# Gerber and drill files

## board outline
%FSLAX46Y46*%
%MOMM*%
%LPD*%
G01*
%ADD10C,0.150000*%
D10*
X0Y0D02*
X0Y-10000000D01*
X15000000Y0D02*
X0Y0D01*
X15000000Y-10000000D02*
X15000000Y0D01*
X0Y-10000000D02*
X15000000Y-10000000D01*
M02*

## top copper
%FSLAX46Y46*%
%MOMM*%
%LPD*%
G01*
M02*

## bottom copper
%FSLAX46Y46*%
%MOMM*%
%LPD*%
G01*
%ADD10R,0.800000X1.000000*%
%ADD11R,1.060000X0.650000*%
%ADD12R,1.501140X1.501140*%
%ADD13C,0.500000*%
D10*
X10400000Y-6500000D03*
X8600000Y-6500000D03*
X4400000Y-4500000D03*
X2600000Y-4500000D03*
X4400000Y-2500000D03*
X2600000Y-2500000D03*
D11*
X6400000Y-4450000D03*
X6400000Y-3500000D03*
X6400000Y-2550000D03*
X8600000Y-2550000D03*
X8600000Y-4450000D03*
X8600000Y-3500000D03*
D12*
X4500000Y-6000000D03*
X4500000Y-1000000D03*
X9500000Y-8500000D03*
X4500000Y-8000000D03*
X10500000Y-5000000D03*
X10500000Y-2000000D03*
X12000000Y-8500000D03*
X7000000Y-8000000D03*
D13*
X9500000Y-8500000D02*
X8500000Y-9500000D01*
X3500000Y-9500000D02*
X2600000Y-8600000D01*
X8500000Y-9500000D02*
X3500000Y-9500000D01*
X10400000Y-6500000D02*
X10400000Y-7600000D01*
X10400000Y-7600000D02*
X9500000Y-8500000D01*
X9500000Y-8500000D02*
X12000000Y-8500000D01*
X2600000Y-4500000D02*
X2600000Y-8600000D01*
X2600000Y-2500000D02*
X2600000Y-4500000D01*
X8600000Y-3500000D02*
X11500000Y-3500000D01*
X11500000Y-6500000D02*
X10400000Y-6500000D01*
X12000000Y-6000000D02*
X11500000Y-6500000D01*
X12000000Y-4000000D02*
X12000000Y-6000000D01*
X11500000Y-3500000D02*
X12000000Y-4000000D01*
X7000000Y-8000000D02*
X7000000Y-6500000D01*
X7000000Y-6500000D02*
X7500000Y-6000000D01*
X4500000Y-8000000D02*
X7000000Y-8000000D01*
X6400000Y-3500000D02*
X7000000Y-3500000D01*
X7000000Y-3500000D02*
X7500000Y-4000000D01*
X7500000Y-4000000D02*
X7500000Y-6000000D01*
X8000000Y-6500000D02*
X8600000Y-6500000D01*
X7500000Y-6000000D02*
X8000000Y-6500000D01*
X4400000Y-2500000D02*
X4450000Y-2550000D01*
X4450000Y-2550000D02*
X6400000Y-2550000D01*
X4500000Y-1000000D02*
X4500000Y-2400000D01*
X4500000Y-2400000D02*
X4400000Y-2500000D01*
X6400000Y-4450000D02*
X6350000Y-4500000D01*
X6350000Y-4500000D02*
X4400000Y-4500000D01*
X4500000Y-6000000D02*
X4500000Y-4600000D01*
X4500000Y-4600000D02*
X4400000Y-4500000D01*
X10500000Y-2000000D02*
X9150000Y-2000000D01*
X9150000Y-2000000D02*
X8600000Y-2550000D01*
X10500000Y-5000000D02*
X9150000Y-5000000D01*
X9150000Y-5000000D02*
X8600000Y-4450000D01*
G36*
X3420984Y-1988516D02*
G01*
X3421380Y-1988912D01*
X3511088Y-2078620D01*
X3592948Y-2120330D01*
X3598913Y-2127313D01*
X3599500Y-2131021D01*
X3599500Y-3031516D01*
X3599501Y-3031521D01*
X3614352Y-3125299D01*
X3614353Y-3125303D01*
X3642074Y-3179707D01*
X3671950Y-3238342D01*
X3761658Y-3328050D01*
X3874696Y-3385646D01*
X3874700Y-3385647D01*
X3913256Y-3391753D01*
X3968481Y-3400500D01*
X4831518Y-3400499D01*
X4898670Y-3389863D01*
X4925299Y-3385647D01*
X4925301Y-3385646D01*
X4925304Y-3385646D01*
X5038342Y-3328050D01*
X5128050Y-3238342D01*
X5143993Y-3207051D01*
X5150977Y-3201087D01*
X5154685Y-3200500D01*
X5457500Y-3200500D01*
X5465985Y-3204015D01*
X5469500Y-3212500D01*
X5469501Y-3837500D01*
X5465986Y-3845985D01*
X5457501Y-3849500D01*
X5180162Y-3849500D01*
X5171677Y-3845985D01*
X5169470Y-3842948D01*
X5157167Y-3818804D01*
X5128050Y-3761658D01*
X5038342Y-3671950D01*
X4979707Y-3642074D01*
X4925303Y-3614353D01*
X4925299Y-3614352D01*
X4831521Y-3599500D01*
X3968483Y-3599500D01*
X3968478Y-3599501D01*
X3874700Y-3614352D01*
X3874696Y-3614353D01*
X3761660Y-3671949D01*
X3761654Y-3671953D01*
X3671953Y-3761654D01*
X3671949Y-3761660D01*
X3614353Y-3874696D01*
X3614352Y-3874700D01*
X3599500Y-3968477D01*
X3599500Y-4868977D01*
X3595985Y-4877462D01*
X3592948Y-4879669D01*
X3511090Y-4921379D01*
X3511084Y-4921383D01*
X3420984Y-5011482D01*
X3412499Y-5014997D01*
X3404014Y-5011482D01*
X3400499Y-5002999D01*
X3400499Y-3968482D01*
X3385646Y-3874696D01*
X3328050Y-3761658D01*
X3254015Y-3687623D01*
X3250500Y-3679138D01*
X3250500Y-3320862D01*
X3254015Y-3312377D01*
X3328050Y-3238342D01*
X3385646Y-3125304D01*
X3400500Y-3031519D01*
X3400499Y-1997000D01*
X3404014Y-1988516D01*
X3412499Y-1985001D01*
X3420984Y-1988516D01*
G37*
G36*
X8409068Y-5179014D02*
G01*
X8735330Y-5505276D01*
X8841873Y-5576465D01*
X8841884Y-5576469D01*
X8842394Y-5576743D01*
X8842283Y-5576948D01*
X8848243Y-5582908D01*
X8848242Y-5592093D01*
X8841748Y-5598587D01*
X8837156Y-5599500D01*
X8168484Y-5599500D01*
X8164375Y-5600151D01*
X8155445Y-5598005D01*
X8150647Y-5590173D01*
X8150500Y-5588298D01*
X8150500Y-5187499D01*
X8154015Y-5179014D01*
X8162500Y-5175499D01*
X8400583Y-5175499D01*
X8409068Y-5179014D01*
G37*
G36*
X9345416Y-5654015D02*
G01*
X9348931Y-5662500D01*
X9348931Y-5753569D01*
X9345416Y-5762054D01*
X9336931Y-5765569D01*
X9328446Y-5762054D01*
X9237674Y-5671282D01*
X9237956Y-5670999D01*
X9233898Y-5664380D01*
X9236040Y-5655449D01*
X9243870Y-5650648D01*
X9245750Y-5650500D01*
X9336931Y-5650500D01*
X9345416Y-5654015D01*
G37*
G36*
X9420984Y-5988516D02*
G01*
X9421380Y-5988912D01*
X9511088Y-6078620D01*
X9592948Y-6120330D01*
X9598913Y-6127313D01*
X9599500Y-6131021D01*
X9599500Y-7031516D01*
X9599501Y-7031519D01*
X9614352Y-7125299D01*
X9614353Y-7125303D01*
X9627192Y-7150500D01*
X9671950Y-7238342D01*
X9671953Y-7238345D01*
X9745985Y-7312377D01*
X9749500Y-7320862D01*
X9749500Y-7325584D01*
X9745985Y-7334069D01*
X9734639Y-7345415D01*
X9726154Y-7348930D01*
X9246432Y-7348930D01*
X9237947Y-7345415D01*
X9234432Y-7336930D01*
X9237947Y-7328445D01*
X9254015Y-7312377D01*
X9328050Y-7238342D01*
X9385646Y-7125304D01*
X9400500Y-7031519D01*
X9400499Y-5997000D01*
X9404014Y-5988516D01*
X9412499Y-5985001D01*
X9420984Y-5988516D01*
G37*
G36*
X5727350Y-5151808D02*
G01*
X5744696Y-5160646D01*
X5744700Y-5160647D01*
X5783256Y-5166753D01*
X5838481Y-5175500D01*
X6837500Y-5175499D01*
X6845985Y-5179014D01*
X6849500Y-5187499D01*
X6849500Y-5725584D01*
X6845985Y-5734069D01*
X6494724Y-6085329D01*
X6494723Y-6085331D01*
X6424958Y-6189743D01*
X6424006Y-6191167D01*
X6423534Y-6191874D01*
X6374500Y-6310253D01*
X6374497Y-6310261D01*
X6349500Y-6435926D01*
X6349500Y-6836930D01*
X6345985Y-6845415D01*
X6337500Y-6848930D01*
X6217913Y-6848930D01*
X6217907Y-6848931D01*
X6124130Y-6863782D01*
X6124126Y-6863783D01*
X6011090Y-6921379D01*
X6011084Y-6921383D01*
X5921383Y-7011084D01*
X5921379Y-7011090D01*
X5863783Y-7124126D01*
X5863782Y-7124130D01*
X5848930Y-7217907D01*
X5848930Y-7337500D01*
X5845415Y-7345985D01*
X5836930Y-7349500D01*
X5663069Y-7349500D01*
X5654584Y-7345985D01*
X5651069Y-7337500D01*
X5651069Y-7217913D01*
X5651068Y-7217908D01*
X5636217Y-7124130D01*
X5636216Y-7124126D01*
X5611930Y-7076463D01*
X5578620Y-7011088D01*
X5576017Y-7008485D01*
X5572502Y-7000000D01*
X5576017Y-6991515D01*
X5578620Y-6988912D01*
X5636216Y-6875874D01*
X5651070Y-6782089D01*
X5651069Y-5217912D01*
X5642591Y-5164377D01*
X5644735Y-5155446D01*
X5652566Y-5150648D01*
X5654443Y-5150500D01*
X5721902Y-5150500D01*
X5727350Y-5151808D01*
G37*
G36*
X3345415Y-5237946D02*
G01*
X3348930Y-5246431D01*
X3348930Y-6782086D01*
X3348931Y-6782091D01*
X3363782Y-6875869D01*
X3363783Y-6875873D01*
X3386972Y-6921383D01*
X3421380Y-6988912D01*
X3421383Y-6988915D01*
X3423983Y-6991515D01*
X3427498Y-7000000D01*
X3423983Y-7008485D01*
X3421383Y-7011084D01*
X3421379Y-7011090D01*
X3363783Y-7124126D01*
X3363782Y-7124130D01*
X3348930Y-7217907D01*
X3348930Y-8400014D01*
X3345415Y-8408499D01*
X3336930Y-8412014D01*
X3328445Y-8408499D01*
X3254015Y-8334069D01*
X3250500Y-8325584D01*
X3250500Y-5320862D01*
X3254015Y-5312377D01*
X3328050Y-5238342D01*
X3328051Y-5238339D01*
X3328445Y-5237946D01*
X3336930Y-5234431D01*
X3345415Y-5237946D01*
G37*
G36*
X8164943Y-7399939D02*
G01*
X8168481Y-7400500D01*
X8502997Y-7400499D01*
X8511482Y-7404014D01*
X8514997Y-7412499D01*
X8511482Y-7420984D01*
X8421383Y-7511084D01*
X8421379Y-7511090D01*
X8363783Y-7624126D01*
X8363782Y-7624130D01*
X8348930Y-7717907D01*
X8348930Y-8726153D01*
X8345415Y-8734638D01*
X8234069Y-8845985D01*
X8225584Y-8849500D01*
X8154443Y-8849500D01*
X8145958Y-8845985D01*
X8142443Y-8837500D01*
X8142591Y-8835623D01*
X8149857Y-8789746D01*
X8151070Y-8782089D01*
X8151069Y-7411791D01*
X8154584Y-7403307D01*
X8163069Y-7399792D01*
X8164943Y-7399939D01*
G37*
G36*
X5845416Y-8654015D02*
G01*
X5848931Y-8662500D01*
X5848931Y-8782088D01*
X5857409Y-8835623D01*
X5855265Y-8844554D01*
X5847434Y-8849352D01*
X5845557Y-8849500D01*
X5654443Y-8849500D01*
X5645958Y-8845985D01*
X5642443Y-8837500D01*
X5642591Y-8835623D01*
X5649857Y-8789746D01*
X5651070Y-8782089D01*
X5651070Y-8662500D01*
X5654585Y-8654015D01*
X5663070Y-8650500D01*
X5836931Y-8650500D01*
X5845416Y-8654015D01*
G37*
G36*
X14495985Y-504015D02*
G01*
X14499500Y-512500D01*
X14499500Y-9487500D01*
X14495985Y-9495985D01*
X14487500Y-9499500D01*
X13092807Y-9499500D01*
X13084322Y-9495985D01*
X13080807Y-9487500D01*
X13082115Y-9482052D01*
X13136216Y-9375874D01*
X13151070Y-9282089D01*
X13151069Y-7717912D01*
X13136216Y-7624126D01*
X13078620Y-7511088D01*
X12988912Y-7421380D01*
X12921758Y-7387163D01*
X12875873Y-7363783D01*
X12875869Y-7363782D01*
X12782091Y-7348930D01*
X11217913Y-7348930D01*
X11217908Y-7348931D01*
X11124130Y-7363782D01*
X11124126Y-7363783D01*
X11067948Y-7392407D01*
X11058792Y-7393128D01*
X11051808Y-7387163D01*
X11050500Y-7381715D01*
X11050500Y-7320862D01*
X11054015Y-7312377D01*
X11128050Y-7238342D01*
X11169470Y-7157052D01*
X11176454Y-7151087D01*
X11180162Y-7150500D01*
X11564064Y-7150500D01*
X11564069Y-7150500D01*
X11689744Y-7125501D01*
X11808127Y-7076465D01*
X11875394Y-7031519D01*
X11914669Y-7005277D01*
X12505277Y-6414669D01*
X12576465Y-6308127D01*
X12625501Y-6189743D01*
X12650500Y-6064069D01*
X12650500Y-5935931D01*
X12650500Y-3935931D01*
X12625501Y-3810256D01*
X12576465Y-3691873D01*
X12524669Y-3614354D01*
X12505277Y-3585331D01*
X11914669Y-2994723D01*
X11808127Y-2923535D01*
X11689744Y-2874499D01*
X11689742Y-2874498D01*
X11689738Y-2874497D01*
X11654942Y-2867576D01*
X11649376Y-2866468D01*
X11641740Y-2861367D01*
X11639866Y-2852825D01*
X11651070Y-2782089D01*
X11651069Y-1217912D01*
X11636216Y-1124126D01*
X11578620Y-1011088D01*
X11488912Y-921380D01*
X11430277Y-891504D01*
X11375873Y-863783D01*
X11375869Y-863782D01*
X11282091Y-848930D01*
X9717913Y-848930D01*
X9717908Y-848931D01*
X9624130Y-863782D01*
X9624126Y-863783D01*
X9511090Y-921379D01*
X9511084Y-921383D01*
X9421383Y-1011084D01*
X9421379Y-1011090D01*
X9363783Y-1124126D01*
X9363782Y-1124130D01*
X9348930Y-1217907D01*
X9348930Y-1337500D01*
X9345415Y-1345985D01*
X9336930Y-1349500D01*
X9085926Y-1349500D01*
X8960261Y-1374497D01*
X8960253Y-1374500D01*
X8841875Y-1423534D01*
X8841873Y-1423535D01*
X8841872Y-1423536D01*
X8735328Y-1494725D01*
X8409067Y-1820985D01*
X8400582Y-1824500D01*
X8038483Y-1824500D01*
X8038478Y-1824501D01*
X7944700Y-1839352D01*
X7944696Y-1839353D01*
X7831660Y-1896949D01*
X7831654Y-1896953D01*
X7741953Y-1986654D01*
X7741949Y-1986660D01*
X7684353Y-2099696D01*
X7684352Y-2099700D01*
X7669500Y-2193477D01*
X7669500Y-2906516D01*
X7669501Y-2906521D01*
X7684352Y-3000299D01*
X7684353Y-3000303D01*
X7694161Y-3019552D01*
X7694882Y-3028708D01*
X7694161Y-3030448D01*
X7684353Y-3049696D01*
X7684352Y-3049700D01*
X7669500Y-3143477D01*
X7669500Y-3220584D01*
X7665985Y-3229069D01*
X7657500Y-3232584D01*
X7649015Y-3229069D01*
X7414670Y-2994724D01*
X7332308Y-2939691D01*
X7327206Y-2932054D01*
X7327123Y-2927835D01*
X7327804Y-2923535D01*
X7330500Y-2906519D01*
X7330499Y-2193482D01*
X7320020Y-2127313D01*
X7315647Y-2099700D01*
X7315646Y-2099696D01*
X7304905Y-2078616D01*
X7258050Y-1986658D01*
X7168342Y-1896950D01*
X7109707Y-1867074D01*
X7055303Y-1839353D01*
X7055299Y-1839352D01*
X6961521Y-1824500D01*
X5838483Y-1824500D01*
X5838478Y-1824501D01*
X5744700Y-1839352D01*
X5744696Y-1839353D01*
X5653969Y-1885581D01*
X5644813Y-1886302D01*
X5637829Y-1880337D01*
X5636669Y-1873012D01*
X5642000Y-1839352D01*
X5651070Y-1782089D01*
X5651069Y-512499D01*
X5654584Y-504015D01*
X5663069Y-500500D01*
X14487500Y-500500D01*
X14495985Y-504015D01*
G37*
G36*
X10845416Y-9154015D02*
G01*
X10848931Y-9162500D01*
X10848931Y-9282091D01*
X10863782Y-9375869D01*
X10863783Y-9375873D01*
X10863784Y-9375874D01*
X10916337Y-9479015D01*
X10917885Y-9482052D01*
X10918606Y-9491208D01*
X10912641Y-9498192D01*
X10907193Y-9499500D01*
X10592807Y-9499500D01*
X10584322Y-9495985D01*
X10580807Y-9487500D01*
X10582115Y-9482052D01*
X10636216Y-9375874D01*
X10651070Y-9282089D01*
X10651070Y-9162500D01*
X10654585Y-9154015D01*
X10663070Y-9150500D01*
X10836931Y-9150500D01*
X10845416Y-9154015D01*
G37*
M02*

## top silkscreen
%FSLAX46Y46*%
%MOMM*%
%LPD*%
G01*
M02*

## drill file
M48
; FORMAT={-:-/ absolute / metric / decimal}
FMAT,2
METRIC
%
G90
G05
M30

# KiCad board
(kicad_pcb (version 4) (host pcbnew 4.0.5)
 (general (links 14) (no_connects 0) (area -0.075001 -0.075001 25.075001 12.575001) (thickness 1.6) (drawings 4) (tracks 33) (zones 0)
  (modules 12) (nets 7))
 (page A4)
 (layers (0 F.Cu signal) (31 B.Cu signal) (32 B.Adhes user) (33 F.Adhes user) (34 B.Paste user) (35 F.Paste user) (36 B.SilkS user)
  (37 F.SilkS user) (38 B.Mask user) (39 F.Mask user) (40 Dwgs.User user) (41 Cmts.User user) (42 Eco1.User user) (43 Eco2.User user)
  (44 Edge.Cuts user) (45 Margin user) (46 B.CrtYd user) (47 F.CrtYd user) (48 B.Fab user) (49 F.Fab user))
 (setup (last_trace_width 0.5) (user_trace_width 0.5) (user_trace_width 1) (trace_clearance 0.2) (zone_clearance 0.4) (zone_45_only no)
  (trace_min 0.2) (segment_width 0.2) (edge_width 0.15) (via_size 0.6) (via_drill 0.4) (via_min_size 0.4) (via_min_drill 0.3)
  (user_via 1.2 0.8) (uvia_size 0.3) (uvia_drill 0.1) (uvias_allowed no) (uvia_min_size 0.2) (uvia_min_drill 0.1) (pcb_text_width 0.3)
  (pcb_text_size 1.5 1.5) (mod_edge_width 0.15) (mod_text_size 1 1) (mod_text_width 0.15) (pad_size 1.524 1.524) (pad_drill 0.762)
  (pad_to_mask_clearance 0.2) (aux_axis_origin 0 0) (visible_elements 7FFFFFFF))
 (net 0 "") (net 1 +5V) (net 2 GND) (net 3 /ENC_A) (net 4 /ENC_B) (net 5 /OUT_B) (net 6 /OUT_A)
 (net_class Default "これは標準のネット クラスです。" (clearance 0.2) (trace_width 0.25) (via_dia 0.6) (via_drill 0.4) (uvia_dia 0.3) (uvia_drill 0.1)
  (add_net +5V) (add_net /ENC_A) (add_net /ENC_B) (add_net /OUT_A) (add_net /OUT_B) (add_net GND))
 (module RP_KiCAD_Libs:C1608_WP (layer B.Cu) (at 9.5 6.5 180)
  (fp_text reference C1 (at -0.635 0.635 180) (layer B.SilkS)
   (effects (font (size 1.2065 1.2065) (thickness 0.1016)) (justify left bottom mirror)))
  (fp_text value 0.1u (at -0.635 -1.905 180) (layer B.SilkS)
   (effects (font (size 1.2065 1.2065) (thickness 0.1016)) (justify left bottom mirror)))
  (pad 1 smd rect (at -0.9 0 180) (size 0.8 1) (layers B.Cu B.Paste B.Mask) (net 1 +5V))
  (pad 2 smd rect (at 0.9 0 180) (size 0.8 1) (layers B.Cu B.Paste B.Mask) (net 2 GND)))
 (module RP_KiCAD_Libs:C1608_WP (layer B.Cu) (at 3.5 4.5 180)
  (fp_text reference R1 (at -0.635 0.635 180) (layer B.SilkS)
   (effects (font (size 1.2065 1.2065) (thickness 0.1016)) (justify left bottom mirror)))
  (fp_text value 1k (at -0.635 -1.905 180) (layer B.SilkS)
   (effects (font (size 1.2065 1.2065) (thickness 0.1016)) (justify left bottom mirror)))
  (pad 1 smd rect (at -0.9 0 180) (size 0.8 1) (layers B.Cu B.Paste B.Mask) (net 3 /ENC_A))
  (pad 2 smd rect (at 0.9 0 180) (size 0.8 1) (layers B.Cu B.Paste B.Mask) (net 1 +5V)))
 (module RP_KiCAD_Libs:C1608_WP (layer B.Cu) (at 3.5 2.5 180)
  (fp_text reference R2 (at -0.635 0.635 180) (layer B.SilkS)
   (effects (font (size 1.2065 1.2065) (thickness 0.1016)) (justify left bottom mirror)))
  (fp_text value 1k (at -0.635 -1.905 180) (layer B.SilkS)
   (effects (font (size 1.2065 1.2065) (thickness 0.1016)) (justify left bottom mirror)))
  (pad 1 smd rect (at -0.9 0 180) (size 0.8 1) (layers B.Cu B.Paste B.Mask) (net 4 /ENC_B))
  (pad 2 smd rect (at 0.9 0 180) (size 0.8 1) (layers B.Cu B.Paste B.Mask) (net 1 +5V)))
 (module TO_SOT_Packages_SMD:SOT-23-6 (layer B.Cu) (at 7.5 3.5)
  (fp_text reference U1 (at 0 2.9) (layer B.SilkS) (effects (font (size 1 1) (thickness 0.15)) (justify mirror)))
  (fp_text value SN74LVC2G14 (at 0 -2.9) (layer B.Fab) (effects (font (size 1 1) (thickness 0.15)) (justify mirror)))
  (pad 1 smd rect (at -1.1 0.95) (size 1.06 0.65) (layers B.Cu B.Paste B.Mask) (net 3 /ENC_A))
  (pad 2 smd rect (at -1.1 0) (size 1.06 0.65) (layers B.Cu B.Paste B.Mask) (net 2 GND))
  (pad 3 smd rect (at -1.1 -0.95) (size 1.06 0.65) (layers B.Cu B.Paste B.Mask) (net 4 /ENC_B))
  (pad 4 smd rect (at 1.1 -0.95) (size 1.06 0.65) (layers B.Cu B.Paste B.Mask) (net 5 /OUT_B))
  (pad 6 smd rect (at 1.1 0.95) (size 1.06 0.65) (layers B.Cu B.Paste B.Mask) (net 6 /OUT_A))
  (pad 5 smd rect (at 1.1 0) (size 1.06 0.65) (layers B.Cu B.Paste B.Mask) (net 1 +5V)))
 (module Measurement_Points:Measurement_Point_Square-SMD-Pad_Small (layer B.Cu) (at 4.5 6 90)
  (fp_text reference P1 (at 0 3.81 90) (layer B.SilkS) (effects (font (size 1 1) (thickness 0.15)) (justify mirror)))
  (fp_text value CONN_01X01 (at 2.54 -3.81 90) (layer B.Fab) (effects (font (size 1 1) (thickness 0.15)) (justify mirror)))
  (pad 1 smd rect (at 0 0 90) (size 1.50114 1.50114) (layers B.Cu B.Paste B.Mask) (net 3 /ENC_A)))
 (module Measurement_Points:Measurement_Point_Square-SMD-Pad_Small (layer B.Cu) (at 4.5 1 270)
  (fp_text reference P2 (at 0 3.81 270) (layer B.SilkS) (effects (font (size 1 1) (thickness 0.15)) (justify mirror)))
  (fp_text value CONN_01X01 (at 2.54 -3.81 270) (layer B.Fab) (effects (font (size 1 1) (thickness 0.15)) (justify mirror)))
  (pad 1 smd rect (at 0 0 270) (size 1.50114 1.50114) (layers B.Cu B.Paste B.Mask) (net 4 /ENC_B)))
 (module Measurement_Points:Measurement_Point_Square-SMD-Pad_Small (layer B.Cu) (at 9.5 8.5)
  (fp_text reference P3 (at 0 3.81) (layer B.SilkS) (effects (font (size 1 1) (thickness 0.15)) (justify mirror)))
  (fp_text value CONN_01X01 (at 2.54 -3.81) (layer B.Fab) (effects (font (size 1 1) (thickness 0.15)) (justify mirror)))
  (pad 1 smd rect (at 0 0) (size 1.50114 1.50114) (layers B.Cu B.Paste B.Mask) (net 1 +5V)))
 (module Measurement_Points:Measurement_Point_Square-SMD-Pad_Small (layer B.Cu) (at 4.5 8)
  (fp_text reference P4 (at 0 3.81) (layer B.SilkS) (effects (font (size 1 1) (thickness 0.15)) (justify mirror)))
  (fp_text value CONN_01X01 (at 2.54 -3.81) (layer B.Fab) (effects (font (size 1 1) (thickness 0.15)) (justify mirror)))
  (pad 1 smd rect (at 0 0) (size 1.50114 1.50114) (layers B.Cu B.Paste B.Mask) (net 2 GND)))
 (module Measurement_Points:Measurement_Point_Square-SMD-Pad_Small (layer B.Cu) (at 10.5 5)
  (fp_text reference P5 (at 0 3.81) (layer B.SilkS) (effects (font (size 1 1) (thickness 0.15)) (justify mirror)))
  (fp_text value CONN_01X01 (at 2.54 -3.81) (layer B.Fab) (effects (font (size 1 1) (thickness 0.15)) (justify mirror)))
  (pad 1 smd rect (at 0 0) (size 1.50114 1.50114) (layers B.Cu B.Paste B.Mask) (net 6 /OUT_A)))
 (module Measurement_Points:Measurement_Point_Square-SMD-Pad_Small (layer B.Cu) (at 10.5 2)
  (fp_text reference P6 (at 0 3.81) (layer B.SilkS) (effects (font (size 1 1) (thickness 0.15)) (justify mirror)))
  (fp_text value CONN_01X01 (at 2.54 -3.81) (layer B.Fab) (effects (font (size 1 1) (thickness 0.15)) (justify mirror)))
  (pad 1 smd rect (at 0 0) (size 1.50114 1.50114) (layers B.Cu B.Paste B.Mask) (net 5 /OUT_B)))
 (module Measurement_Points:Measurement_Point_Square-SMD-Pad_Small (layer B.Cu) (at 12 8.5)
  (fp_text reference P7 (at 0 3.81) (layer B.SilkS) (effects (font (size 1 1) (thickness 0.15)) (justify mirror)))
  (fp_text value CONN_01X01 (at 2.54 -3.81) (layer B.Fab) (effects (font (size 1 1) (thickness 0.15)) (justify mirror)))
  (pad 1 smd rect (at 0 0) (size 1.50114 1.50114) (layers B.Cu B.Paste B.Mask) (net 1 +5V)))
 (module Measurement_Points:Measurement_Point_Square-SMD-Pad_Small (layer B.Cu) (at 7 8)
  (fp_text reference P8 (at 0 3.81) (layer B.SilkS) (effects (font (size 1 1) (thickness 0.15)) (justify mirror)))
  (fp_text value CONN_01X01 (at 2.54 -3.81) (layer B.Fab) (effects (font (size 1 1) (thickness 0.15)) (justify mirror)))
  (pad 1 smd rect (at 0 0) (size 1.50114 1.50114) (layers B.Cu B.Paste B.Mask) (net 2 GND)))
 (gr_line (start 0 0) (end 0 10) (angle 90) (layer Edge.Cuts) (width 0.15))
 (gr_line (start 15 0) (end 0 0) (angle 90) (layer Edge.Cuts) (width 0.15))
 (gr_line (start 15 10) (end 15 0) (angle 90) (layer Edge.Cuts) (width 0.15))
 (gr_line (start 0 10) (end 15 10) (angle 90) (layer Edge.Cuts) (width 0.15))
 (segment (start 9.5 8.5) (end 8.5 9.5) (width 0.5) (layer B.Cu) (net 1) (status 400000))
 (segment (start 3.5 9.5) (end 2.6 8.6) (width 0.5) (layer B.Cu) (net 1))
 (segment (start 8.5 9.5) (end 3.5 9.5) (width 0.5) (layer B.Cu) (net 1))
 (segment (start 10.4 6.5) (end 10.4 7.6) (width 0.5) (layer B.Cu) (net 1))
 (segment (start 10.4 7.6) (end 9.5 8.5) (width 0.5) (layer B.Cu) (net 1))
 (segment (start 9.5 8.5) (end 12 8.5) (width 0.5) (layer B.Cu) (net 1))
 (segment (start 2.6 4.5) (end 2.6 8.6) (width 0.5) (layer B.Cu) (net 1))
 (segment (start 2.6 2.5) (end 2.6 4.5) (width 0.5) (layer B.Cu) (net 1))
 (segment (start 8.6 3.5) (end 11.5 3.5) (width 0.5) (layer B.Cu) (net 1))
 (segment (start 11.5 6.5) (end 10.4 6.5) (width 0.5) (layer B.Cu) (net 1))
 (segment (start 12 6) (end 11.5 6.5) (width 0.5) (layer B.Cu) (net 1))
 (segment (start 12 4) (end 12 6) (width 0.5) (layer B.Cu) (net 1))
 (segment (start 11.5 3.5) (end 12 4) (width 0.5) (layer B.Cu) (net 1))
 (segment (start 7 8) (end 7 6.5) (width 0.5) (layer B.Cu) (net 2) (status 400000))
 (segment (start 7 6.5) (end 7.5 6) (width 0.5) (layer B.Cu) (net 2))
 (segment (start 4.5 8) (end 7 8) (width 0.5) (layer B.Cu) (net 2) (status C00000))
 (segment (start 6.4 3.5) (end 7 3.5) (width 0.5) (layer B.Cu) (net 2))
 (segment (start 7 3.5) (end 7.5 4) (width 0.5) (layer B.Cu) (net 2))
 (segment (start 7.5 4) (end 7.5 6) (width 0.5) (layer B.Cu) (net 2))
 (segment (start 8 6.5) (end 8.6 6.5) (width 0.5) (layer B.Cu) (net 2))
 (segment (start 7.5 6) (end 8 6.5) (width 0.5) (layer B.Cu) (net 2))
 (segment (start 4.4 2.5) (end 4.45 2.55) (width 0.5) (layer B.Cu) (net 4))
 (segment (start 4.45 2.55) (end 6.4 2.55) (width 0.5) (layer B.Cu) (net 4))
 (segment (start 4.5 1) (end 4.5 2.4) (width 0.5) (layer B.Cu) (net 4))
 (segment (start 4.5 2.4) (end 4.4 2.5) (width 0.5) (layer B.Cu) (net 4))
 (segment (start 6.4 4.45) (end 6.35 4.5) (width 0.5) (layer B.Cu) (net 3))
 (segment (start 6.35 4.5) (end 4.4 4.5) (width 0.5) (layer B.Cu) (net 3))
 (segment (start 4.5 6) (end 4.5 4.6) (width 0.5) (layer B.Cu) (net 3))
 (segment (start 4.5 4.6) (end 4.4 4.5) (width 0.5) (layer B.Cu) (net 3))
 (segment (start 10.5 2) (end 9.15 2) (width 0.5) (layer B.Cu) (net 5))
 (segment (start 9.15 2) (end 8.6 2.55) (width 0.5) (layer B.Cu) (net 5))
 (segment (start 10.5 5) (end 9.15 5) (width 0.5) (layer B.Cu) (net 6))
 (segment (start 9.15 5) (end 8.6 4.45) (width 0.5) (layer B.Cu) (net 6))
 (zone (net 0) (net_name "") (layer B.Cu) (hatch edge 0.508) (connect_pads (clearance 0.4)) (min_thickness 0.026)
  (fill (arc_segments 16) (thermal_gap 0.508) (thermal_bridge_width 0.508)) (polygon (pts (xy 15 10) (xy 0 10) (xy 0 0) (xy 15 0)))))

